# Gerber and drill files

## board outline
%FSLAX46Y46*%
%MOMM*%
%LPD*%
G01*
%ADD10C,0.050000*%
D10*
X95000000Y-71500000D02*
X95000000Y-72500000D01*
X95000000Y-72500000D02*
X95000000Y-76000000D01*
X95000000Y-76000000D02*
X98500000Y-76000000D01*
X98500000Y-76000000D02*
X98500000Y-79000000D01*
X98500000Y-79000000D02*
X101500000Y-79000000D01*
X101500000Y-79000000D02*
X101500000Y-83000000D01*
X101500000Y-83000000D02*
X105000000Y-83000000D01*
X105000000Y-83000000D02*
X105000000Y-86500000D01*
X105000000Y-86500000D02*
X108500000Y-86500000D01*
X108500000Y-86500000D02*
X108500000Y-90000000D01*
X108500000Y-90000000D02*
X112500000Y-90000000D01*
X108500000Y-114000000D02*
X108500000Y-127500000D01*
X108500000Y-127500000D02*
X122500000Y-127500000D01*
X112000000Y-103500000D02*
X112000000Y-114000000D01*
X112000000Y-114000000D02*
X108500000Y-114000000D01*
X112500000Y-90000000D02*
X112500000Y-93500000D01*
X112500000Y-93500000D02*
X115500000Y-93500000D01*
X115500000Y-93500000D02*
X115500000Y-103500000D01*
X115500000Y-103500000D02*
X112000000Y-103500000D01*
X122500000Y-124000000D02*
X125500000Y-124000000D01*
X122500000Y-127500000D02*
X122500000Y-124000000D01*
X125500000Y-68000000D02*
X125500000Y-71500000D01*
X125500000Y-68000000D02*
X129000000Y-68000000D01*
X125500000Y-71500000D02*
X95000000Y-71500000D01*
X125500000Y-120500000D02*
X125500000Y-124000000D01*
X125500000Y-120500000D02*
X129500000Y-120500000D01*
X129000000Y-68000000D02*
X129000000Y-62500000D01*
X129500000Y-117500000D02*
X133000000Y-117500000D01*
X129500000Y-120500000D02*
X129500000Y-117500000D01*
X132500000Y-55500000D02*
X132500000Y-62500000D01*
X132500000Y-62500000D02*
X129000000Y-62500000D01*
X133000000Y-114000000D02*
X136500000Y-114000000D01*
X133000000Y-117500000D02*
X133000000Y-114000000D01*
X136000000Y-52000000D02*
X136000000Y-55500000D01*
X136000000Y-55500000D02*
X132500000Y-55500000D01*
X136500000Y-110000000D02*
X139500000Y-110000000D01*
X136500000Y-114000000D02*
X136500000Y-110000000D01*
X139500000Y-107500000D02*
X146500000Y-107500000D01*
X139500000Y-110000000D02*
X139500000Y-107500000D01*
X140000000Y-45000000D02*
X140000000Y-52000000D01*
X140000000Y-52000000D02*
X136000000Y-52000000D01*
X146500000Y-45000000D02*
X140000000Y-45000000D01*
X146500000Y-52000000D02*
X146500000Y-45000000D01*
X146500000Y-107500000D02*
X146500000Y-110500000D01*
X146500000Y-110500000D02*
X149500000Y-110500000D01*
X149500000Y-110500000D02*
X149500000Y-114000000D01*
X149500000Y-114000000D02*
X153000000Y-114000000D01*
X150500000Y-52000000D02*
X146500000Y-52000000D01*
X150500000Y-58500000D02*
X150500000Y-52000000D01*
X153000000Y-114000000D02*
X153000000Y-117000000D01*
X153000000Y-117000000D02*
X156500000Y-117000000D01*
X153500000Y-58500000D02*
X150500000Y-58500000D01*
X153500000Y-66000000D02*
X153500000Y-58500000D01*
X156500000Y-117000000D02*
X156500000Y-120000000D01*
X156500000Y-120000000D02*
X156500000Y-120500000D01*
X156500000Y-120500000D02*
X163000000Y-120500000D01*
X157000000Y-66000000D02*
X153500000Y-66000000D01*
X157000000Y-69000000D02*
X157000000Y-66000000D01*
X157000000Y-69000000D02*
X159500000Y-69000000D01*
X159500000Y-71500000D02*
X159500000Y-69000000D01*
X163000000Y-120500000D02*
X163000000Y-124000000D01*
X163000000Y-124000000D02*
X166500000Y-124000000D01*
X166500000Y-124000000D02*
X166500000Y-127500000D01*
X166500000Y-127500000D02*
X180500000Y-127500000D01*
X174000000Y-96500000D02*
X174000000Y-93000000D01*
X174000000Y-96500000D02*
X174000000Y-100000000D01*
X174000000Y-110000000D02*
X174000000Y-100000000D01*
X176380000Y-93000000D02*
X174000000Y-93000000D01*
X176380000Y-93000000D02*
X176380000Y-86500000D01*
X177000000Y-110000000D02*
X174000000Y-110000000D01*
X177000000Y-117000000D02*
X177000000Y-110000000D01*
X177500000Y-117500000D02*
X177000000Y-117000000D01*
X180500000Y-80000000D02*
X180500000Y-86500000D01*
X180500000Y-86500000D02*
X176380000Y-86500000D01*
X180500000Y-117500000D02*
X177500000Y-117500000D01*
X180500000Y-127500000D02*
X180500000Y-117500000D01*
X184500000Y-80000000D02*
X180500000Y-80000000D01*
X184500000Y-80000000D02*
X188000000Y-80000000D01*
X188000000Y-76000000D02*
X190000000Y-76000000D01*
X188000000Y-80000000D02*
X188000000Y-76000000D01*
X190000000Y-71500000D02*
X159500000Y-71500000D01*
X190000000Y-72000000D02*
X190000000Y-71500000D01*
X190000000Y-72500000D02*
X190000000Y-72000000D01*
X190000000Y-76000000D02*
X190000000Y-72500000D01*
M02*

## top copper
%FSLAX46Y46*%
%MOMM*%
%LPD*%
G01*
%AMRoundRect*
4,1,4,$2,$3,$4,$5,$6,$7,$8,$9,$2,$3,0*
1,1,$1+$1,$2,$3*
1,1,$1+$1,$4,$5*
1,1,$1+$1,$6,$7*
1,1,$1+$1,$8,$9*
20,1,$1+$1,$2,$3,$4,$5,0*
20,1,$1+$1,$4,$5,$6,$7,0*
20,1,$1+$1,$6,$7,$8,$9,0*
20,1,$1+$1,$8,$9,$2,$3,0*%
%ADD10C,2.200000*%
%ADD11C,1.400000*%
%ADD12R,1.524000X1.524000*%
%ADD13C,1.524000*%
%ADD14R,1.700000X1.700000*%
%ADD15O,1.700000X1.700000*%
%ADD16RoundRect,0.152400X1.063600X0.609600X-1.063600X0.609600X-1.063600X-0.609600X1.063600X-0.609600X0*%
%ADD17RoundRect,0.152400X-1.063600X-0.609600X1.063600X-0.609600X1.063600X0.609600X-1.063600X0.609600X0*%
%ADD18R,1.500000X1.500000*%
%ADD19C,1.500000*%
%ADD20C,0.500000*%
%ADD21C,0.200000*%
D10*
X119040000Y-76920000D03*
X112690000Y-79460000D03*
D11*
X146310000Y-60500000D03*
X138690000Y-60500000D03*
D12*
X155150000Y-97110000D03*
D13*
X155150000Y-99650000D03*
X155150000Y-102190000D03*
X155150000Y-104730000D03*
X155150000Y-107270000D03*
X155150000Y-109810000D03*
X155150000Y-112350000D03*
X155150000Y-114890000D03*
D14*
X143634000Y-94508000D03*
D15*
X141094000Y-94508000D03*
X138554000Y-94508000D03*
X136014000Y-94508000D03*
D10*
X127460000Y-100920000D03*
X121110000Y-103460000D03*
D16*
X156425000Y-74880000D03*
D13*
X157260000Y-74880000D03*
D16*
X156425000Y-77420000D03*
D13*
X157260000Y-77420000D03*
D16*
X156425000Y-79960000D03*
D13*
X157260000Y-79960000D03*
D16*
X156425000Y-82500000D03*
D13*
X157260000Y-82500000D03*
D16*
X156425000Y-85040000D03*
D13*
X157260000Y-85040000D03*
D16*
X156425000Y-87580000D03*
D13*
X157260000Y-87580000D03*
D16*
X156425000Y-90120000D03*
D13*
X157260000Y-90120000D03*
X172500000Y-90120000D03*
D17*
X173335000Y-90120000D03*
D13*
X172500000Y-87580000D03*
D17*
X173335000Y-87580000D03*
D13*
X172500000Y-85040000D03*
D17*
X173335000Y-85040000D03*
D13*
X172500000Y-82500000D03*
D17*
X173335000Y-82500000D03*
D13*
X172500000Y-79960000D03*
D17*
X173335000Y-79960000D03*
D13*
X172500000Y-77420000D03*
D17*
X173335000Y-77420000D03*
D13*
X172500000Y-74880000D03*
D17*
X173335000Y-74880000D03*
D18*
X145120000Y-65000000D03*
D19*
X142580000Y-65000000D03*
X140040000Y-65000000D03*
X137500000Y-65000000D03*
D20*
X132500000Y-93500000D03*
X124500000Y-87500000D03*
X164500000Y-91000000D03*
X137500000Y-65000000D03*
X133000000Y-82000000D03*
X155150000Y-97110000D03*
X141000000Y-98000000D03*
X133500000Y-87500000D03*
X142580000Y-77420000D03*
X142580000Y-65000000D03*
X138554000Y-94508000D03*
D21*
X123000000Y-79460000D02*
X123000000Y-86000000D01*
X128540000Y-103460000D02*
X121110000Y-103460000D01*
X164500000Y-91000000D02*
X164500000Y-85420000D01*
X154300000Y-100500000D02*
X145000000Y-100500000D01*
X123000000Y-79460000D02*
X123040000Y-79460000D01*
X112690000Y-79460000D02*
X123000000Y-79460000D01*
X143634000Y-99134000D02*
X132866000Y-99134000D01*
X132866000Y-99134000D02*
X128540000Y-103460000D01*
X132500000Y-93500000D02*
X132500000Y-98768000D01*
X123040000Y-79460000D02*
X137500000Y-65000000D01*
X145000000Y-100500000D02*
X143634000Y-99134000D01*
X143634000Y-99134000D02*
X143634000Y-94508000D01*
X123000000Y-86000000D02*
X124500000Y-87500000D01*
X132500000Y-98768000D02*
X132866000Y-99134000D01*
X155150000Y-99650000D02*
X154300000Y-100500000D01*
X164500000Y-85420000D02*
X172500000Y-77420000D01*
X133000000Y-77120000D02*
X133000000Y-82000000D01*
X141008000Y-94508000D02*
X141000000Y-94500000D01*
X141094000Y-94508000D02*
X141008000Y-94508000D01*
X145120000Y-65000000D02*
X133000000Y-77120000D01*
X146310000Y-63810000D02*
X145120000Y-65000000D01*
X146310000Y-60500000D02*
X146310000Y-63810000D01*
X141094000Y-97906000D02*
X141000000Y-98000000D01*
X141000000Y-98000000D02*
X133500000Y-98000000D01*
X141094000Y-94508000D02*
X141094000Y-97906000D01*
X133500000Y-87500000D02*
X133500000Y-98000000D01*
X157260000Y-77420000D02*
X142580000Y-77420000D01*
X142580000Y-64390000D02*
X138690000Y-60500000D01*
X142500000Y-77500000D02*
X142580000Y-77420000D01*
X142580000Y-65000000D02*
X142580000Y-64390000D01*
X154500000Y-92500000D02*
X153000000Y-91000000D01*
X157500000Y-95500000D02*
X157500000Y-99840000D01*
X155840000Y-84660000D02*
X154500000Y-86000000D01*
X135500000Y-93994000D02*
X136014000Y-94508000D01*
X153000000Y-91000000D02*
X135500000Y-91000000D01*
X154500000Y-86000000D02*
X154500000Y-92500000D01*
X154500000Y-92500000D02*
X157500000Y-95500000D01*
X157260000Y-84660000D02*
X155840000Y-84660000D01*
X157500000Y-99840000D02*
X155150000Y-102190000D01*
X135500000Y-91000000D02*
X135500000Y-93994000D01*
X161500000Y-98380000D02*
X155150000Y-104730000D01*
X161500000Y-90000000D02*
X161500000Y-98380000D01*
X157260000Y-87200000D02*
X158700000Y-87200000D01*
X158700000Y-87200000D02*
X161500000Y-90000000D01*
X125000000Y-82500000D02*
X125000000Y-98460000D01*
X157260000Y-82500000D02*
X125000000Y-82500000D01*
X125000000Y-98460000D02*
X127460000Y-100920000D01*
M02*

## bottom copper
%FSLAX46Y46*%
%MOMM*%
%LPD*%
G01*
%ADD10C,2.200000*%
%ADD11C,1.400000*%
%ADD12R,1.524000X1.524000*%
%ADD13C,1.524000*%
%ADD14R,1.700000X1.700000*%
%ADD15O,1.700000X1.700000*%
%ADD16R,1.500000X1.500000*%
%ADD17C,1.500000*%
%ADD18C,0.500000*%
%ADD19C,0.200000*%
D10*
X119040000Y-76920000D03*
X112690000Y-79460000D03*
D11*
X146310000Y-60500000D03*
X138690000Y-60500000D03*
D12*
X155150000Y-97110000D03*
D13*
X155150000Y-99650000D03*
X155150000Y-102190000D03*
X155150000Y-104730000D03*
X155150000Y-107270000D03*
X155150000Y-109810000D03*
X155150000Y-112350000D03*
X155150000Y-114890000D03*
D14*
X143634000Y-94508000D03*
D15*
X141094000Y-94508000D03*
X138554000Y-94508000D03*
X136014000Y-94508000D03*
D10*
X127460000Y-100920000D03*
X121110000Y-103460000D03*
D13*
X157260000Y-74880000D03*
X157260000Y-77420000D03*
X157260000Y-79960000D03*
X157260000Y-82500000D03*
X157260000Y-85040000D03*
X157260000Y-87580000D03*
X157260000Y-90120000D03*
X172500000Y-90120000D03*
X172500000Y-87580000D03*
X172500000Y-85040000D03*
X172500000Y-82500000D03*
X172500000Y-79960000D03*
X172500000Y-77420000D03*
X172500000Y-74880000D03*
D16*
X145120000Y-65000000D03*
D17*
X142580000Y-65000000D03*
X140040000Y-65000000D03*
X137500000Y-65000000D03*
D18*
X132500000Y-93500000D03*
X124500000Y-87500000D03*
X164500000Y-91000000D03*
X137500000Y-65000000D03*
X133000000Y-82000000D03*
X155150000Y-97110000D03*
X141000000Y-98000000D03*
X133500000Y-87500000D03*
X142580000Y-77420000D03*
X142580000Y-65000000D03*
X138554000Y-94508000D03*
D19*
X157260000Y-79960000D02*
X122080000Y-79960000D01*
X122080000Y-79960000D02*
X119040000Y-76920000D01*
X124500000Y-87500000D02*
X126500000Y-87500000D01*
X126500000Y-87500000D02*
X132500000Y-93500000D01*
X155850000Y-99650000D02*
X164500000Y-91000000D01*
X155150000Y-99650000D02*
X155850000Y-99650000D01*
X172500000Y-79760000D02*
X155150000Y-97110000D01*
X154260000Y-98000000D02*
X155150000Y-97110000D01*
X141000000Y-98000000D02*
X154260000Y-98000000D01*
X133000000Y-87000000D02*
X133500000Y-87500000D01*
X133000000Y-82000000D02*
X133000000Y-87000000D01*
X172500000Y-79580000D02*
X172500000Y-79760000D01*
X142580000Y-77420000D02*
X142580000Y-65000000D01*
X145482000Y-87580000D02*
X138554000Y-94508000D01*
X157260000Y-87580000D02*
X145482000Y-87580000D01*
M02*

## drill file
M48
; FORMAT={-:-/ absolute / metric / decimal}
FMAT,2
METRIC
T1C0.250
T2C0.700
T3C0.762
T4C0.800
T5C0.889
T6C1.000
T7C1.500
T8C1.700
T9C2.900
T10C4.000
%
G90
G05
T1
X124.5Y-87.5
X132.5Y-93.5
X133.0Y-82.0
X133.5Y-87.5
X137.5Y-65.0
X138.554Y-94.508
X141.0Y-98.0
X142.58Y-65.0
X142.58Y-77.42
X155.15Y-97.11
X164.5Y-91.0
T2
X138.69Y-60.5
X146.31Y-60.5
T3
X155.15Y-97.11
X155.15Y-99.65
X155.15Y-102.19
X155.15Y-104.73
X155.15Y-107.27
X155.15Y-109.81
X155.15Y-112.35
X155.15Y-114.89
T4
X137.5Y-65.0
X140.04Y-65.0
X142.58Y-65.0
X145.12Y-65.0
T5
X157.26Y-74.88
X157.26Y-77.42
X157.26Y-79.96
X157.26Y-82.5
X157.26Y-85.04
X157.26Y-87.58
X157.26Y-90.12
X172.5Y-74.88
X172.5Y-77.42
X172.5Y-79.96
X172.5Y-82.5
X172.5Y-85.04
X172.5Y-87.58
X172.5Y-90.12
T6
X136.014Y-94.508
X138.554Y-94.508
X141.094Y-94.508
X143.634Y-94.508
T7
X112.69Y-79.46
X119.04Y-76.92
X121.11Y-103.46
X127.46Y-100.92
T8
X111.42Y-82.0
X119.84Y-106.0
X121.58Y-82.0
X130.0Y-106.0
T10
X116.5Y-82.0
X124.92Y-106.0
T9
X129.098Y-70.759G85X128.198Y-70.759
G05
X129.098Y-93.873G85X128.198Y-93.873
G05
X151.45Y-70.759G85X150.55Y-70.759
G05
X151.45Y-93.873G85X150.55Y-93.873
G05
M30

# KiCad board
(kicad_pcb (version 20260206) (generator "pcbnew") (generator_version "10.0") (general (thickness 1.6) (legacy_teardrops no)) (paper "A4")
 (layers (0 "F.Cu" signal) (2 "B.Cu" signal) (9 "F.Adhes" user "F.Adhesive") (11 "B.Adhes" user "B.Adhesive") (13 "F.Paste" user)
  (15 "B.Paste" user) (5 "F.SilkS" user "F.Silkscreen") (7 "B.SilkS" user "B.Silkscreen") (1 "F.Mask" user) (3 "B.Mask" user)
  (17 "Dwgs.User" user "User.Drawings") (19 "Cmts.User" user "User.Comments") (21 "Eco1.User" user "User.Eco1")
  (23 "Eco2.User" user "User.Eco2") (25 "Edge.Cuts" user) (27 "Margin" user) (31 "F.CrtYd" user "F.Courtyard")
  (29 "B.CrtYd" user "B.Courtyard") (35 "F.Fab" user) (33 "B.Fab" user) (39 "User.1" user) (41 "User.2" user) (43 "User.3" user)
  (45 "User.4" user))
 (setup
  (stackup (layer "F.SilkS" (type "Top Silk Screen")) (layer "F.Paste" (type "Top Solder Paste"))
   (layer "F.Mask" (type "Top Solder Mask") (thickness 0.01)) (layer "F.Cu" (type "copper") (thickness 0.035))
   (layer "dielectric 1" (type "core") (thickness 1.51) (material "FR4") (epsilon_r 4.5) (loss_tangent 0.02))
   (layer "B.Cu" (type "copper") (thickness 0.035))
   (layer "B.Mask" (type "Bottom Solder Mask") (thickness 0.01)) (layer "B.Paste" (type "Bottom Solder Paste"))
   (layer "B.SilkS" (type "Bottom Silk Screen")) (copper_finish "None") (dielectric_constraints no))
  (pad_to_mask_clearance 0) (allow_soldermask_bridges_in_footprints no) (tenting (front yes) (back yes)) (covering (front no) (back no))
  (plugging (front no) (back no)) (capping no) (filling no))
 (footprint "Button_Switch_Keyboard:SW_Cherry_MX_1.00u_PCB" (layer "F.Cu") (at 119.04 76.92)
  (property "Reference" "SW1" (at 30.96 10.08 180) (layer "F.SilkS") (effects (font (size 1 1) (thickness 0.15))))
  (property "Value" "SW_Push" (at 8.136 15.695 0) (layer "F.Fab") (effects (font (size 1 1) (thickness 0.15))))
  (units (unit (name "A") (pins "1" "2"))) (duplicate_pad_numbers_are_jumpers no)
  (pad "" np_thru_hole circle (at -7.62 5.08) (size 1.7 1.7) (drill 1.7) (layers "*.Cu" "*.Mask"))
  (pad "" np_thru_hole circle (at -2.54 5.08) (size 4 4) (drill 4) (layers "*.Cu" "*.Mask"))
  (pad "" np_thru_hole circle (at 2.54 5.08) (size 1.7 1.7) (drill 1.7) (layers "*.Cu" "*.Mask"))
  (pad "1" thru_hole circle (at 0 0) (size 2.2 2.2) (drill 1.5) (layers "*.Cu" "*.Mask") (remove_unused_layers no) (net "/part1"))
  (pad "2" thru_hole circle (at -6.35 2.54) (size 2.2 2.2) (drill 1.5) (layers "*.Cu" "*.Mask") (remove_unused_layers no) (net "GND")))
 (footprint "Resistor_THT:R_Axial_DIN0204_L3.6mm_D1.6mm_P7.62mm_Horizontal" (layer "F.Cu") (at 146.31 60.5 180)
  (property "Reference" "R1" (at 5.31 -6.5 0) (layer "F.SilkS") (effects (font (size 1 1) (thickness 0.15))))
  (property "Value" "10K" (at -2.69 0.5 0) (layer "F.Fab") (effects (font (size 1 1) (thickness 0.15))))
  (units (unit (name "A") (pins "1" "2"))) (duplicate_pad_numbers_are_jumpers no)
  (pad "1" thru_hole circle (at 0 0 180) (size 1.4 1.4) (drill 0.7) (layers "*.Cu" "*.Mask") (remove_unused_layers no) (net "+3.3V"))
  (pad "2" thru_hole circle (at 7.62 0 180) (size 1.4 1.4) (drill 0.7) (layers "*.Cu" "*.Mask") (remove_unused_layers no)
   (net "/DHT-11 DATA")))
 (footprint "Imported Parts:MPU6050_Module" (layer "F.Cu") (at 155.15 97.11)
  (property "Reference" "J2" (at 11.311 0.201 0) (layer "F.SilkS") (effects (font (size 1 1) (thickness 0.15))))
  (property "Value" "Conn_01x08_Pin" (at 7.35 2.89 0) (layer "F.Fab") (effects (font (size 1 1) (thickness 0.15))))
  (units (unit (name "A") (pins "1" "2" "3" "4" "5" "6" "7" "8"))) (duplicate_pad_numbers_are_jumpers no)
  (pad "1" thru_hole rect (at 0 0) (size 1.524 1.524) (drill 0.762) (layers "*.Cu" "*.Mask") (remove_unused_layers no) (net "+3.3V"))
  (pad "2" thru_hole circle (at 0 2.54) (size 1.524 1.524) (drill 0.762) (layers "*.Cu" "*.Mask") (remove_unused_layers no) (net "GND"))
  (pad "3" thru_hole circle (at 0 5.08) (size 1.524 1.524) (drill 0.762) (layers "*.Cu" "*.Mask") (remove_unused_layers no) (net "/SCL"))
  (pad "4" thru_hole circle (at 0 7.62) (size 1.524 1.524) (drill 0.762) (layers "*.Cu" "*.Mask") (remove_unused_layers no) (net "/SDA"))
  (pad "5" thru_hole circle (at 0 10.16) (size 1.524 1.524) (drill 0.762) (layers "*.Cu" "*.Mask") (remove_unused_layers no)
   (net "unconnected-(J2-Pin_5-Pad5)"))
  (pad "6" thru_hole circle (at 0 12.7) (size 1.524 1.524) (drill 0.762) (layers "*.Cu" "*.Mask") (remove_unused_layers no)
   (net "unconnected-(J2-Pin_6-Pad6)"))
  (pad "7" thru_hole circle (at 0 15.24) (size 1.524 1.524) (drill 0.762) (layers "*.Cu" "*.Mask") (remove_unused_layers no)
   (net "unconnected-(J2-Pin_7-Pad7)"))
  (pad "8" thru_hole circle (at 0 17.78) (size 1.524 1.524) (drill 0.762) (layers "*.Cu" "*.Mask") (remove_unused_layers no)
   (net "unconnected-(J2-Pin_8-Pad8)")))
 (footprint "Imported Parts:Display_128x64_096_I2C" (layer "F.Cu") (at 139.824 94.508 180)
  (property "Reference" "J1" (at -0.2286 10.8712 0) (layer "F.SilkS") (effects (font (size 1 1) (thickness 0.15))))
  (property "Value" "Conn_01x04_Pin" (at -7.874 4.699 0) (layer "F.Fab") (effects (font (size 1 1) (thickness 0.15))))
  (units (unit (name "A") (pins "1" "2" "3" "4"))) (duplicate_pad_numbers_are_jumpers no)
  (pad "" np_thru_hole oval (at -11.176 0.635 180) (size 3.8 2.9) (drill oval 3.8 2.9) (layers "*.Cu" "*.Mask"))
  (pad "" np_thru_hole oval (at -11.176 23.749 180) (size 3.8 2.9) (drill oval 3.8 2.9) (layers "*.Cu" "*.Mask"))
  (pad "" np_thru_hole oval (at 11.176 0.635 180) (size 3.8 2.9) (drill oval 3.8 2.9) (layers "*.Cu" "*.Mask"))
  (pad "" np_thru_hole oval (at 11.176 23.749 180) (size 3.8 2.9) (drill oval 3.8 2.9) (layers "*.Cu" "*.Mask"))
  (pad "1" thru_hole rect (at -3.81 0 270) (size 1.7 1.7) (drill 1) (layers "*.Cu" "*.Mask") (remove_unused_layers no) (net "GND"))
  (pad "2" thru_hole oval (at -1.27 0 270) (size 1.7 1.7) (drill 1) (layers "*.Cu" "*.Mask") (remove_unused_layers no) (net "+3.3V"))
  (pad "3" thru_hole oval (at 1.27 0 270) (size 1.7 1.7) (drill 1) (layers "*.Cu" "*.Mask") (remove_unused_layers no) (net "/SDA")
   (solder_mask_margin 0))
  (pad "4" thru_hole oval (at 3.81 0 270) (size 1.7 1.7) (drill 1) (layers "*.Cu" "*.Mask") (remove_unused_layers no) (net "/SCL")))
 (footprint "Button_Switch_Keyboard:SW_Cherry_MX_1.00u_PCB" (layer "F.Cu") (at 127.46 100.92)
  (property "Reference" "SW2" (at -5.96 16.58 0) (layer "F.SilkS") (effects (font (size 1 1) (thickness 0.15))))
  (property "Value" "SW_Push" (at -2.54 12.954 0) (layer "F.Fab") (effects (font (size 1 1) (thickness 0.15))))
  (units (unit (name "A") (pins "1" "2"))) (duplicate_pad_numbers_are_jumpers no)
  (pad "" np_thru_hole circle (at -7.62 5.08) (size 1.7 1.7) (drill 1.7) (layers "*.Cu" "*.Mask"))
  (pad "" np_thru_hole circle (at -2.54 5.08) (size 4 4) (drill 4) (layers "*.Cu" "*.Mask"))
  (pad "" np_thru_hole circle (at 2.54 5.08) (size 1.7 1.7) (drill 1.7) (layers "*.Cu" "*.Mask"))
  (pad "1" thru_hole circle (at 0 0) (size 2.2 2.2) (drill 1.5) (layers "*.Cu" "*.Mask") (remove_unused_layers no) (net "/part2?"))
  (pad "2" thru_hole circle (at -6.35 2.54) (size 2.2 2.2) (drill 1.5) (layers "*.Cu" "*.Mask") (remove_unused_layers no) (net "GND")))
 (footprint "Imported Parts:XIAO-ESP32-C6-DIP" (layer "F.Cu") (at 164.88 82.5 90)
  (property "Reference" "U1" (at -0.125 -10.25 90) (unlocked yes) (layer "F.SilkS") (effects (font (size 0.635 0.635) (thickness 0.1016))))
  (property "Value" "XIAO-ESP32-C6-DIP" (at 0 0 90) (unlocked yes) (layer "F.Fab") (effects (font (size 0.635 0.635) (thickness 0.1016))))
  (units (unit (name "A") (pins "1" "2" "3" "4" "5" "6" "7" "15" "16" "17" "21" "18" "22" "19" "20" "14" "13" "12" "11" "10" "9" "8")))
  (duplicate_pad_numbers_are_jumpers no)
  (pad "1" smd roundrect (at 7.62 -8.455 180) (size 2.432 1.524) (layers "F.Cu" "F.Mask") (roundrect_rratio 0.1)
   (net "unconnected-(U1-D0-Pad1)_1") (thermal_bridge_angle 45))
  (pad "1" thru_hole circle (at 7.62 -7.62 180) (size 1.524 1.524) (drill 0.889) (layers "*.Cu" "*.Mask") (remove_unused_layers no)
   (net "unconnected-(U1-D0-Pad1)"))
  (pad "2" smd roundrect (at 5.08 -8.455 180) (size 2.432 1.524) (layers "F.Cu" "F.Mask") (roundrect_rratio 0.1) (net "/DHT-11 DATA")
   (thermal_bridge_angle 45))
  (pad "2" thru_hole circle (at 5.08 -7.62 180) (size 1.524 1.524) (drill 0.889) (layers "*.Cu" "*.Mask") (remove_unused_layers no)
   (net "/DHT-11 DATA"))
  (pad "3" smd roundrect (at 2.54 -8.455 180) (size 2.432 1.524) (layers "F.Cu" "F.Mask") (roundrect_rratio 0.1) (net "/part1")
   (thermal_bridge_angle 45))
  (pad "3" thru_hole circle (at 2.54 -7.62 180) (size 1.524 1.524) (drill 0.889) (layers "*.Cu" "*.Mask") (remove_unused_layers no)
   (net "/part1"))
  (pad "4" smd roundrect (at 0 -8.455 180) (size 2.432 1.524) (layers "F.Cu" "F.Mask") (roundrect_rratio 0.1) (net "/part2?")
   (thermal_bridge_angle 45))
  (pad "4" thru_hole circle (at 0 -7.62 180) (size 1.524 1.524) (drill 0.889) (layers "*.Cu" "*.Mask") (remove_unused_layers no)
   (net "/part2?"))
  (pad "5" smd roundrect (at -2.54 -8.455 180) (size 2.432 1.524) (layers "F.Cu" "F.Mask") (roundrect_rratio 0.1) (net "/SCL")
   (thermal_bridge_angle 45))
  (pad "5" thru_hole circle (at -2.54 -7.62 180) (size 1.524 1.524) (drill 0.889) (layers "*.Cu" "*.Mask") (remove_unused_layers no)
   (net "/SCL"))
  (pad "6" smd roundrect (at -5.08 -8.455 180) (size 2.432 1.524) (layers "F.Cu" "F.Mask") (roundrect_rratio 0.1) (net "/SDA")
   (thermal_bridge_angle 45))
  (pad "6" thru_hole circle (at -5.08 -7.62 180) (size 1.524 1.524) (drill 0.889) (layers "*.Cu" "*.Mask") (remove_unused_layers no)
   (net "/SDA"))
  (pad "7" smd roundrect (at -7.62 -8.455 180) (size 2.432 1.524) (layers "F.Cu" "F.Mask") (roundrect_rratio 0.1)
   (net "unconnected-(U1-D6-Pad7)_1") (thermal_bridge_angle 45))
  (pad "7" thru_hole circle (at -7.62 -7.62 180) (size 1.524 1.524) (drill 0.889) (layers "*.Cu" "*.Mask") (remove_unused_layers no)
   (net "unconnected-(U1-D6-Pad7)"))
  (pad "8" thru_hole circle (at -7.62 7.62) (size 1.524 1.524) (drill 0.889) (layers "*.Cu" "*.Mask") (remove_unused_layers no)
   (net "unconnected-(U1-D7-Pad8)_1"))
  (pad "8" smd roundrect (at -7.62 8.455) (size 2.432 1.524) (layers "F.Cu" "F.Mask") (roundrect_rratio 0.1)
   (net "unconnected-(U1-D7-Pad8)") (thermal_bridge_angle 45))
  (pad "9" thru_hole circle (at -5.08 7.62) (size 1.524 1.524) (drill 0.889) (layers "*.Cu" "*.Mask") (remove_unused_layers no)
   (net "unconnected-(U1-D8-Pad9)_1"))
  (pad "9" smd roundrect (at -5.08 8.455) (size 2.432 1.524) (layers "F.Cu" "F.Mask") (roundrect_rratio 0.1)
   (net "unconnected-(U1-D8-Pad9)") (thermal_bridge_angle 45))
  (pad "10" thru_hole circle (at -2.54 7.62) (size 1.524 1.524) (drill 0.889) (layers "*.Cu" "*.Mask") (remove_unused_layers no)
   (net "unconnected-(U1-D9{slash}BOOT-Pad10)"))
  (pad "10" smd roundrect (at -2.54 8.455) (size 2.432 1.524) (layers "F.Cu" "F.Mask") (roundrect_rratio 0.1)
   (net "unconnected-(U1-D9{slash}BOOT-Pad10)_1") (thermal_bridge_angle 45))
  (pad "11" thru_hole circle (at 0 7.62) (size 1.524 1.524) (drill 0.889) (layers "*.Cu" "*.Mask") (remove_unused_layers no)
   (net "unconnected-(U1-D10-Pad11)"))
  (pad "11" smd roundrect (at 0 8.455) (size 2.432 1.524) (layers "F.Cu" "F.Mask") (roundrect_rratio 0.1)
   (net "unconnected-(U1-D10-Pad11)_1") (thermal_bridge_angle 45))
  (pad "12" thru_hole circle (at 2.54 7.62) (size 1.524 1.524) (drill 0.889) (layers "*.Cu" "*.Mask") (remove_unused_layers no)
   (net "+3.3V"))
  (pad "12" smd roundrect (at 2.54 8.455) (size 2.432 1.524) (layers "F.Cu" "F.Mask") (roundrect_rratio 0.1) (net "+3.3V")
   (thermal_bridge_angle 45))
  (pad "13" thru_hole circle (at 5.08 7.62) (size 1.524 1.524) (drill 0.889) (layers "*.Cu" "*.Mask") (remove_unused_layers no) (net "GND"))
  (pad "13" smd roundrect (at 5.08 8.455) (size 2.432 1.524) (layers "F.Cu" "F.Mask") (roundrect_rratio 0.1) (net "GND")
   (thermal_bridge_angle 45))
  (pad "14" thru_hole circle (at 7.62 7.62) (size 1.524 1.524) (drill 0.889) (layers "*.Cu" "*.Mask") (remove_unused_layers no) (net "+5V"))
  (pad "14" smd roundrect (at 7.62 8.455) (size 2.432 1.524) (layers "F.Cu" "F.Mask") (roundrect_rratio 0.1) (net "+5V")
   (thermal_bridge_angle 45)))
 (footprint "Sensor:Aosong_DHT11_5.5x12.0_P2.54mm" (layer "F.Cu") (at 145.12 65 -90)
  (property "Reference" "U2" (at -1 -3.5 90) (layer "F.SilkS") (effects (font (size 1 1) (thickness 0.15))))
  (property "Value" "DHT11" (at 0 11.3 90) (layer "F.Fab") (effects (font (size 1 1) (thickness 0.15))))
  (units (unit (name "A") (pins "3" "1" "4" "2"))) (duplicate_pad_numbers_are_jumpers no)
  (pad "1" thru_hole rect (at 0 0 270) (size 1.5 1.5) (drill 0.8) (layers "*.Cu" "*.Mask") (remove_unused_layers no) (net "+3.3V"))
  (pad "2" thru_hole circle (at 0 2.54 270) (size 1.5 1.5) (drill 0.8) (layers "*.Cu" "*.Mask") (remove_unused_layers no)
   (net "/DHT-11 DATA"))
  (pad "3" thru_hole circle (at 0 5.08 270) (size 1.5 1.5) (drill 0.8) (layers "*.Cu" "*.Mask") (remove_unused_layers no)
   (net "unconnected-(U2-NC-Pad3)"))
  (pad "4" thru_hole circle (at 0 7.62 270) (size 1.5 1.5) (drill 0.8) (layers "*.Cu" "*.Mask") (remove_unused_layers no) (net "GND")))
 (gr_line (start 95 71.5) (end 95 72.5) (stroke (width 0.05) (type default)) (layer "Edge.Cuts"))
 (gr_line (start 95 72.5) (end 95 76) (stroke (width 0.05) (type default)) (layer "Edge.Cuts"))
 (gr_line (start 95 76) (end 98.5 76) (stroke (width 0.05) (type default)) (layer "Edge.Cuts"))
 (gr_line (start 98.5 76) (end 98.5 79) (stroke (width 0.05) (type default)) (layer "Edge.Cuts"))
 (gr_line (start 98.5 79) (end 101.5 79) (stroke (width 0.05) (type default)) (layer "Edge.Cuts"))
 (gr_line (start 101.5 79) (end 101.5 83) (stroke (width 0.05) (type default)) (layer "Edge.Cuts"))
 (gr_line (start 101.5 83) (end 105 83) (stroke (width 0.05) (type default)) (layer "Edge.Cuts"))
 (gr_line (start 105 83) (end 105 86.5) (stroke (width 0.05) (type default)) (layer "Edge.Cuts"))
 (gr_line (start 105 86.5) (end 108.5 86.5) (stroke (width 0.05) (type default)) (layer "Edge.Cuts"))
 (gr_line (start 108.5 86.5) (end 108.5 90) (stroke (width 0.05) (type default)) (layer "Edge.Cuts"))
 (gr_line (start 108.5 90) (end 112.5 90) (stroke (width 0.05) (type default)) (layer "Edge.Cuts"))
 (gr_line (start 108.5 114) (end 108.5 127.5) (stroke (width 0.05) (type default)) (layer "Edge.Cuts"))
 (gr_line (start 108.5 127.5) (end 122.5 127.5) (stroke (width 0.05) (type default)) (layer "Edge.Cuts"))
 (gr_line (start 112 103.5) (end 112 114) (stroke (width 0.05) (type default)) (layer "Edge.Cuts"))
 (gr_line (start 112 114) (end 108.5 114) (stroke (width 0.05) (type default)) (layer "Edge.Cuts"))
 (gr_line (start 112.5 90) (end 112.5 93.5) (stroke (width 0.05) (type default)) (layer "Edge.Cuts"))
 (gr_line (start 112.5 93.5) (end 115.5 93.5) (stroke (width 0.05) (type default)) (layer "Edge.Cuts"))
 (gr_line (start 115.5 93.5) (end 115.5 103.5) (stroke (width 0.05) (type default)) (layer "Edge.Cuts"))
 (gr_line (start 115.5 103.5) (end 112 103.5) (stroke (width 0.05) (type default)) (layer "Edge.Cuts"))
 (gr_line (start 122.5 124) (end 125.5 124) (stroke (width 0.05) (type default)) (layer "Edge.Cuts"))
 (gr_line (start 122.5 127.5) (end 122.5 124) (stroke (width 0.05) (type default)) (layer "Edge.Cuts"))
 (gr_line (start 125.5 68) (end 125.5 71.5) (stroke (width 0.05) (type default)) (layer "Edge.Cuts"))
 (gr_line (start 125.5 68) (end 129 68) (stroke (width 0.05) (type default)) (layer "Edge.Cuts"))
 (gr_line (start 125.5 71.5) (end 95 71.5) (stroke (width 0.05) (type default)) (layer "Edge.Cuts"))
 (gr_line (start 125.5 120.5) (end 125.5 124) (stroke (width 0.05) (type default)) (layer "Edge.Cuts"))
 (gr_line (start 125.5 120.5) (end 129.5 120.5) (stroke (width 0.05) (type default)) (layer "Edge.Cuts"))
 (gr_line (start 129 68) (end 129 62.5) (stroke (width 0.05) (type default)) (layer "Edge.Cuts"))
 (gr_line (start 129.5 117.5) (end 133 117.5) (stroke (width 0.05) (type default)) (layer "Edge.Cuts"))
 (gr_line (start 129.5 120.5) (end 129.5 117.5) (stroke (width 0.05) (type default)) (layer "Edge.Cuts"))
 (gr_line (start 132.5 55.5) (end 132.5 62.5) (stroke (width 0.05) (type default)) (layer "Edge.Cuts"))
 (gr_line (start 132.5 62.5) (end 129 62.5) (stroke (width 0.05) (type default)) (layer "Edge.Cuts"))
 (gr_line (start 133 114) (end 136.5 114) (stroke (width 0.05) (type default)) (layer "Edge.Cuts"))
 (gr_line (start 133 117.5) (end 133 114) (stroke (width 0.05) (type default)) (layer "Edge.Cuts"))
 (gr_line (start 136 52) (end 136 55.5) (stroke (width 0.05) (type default)) (layer "Edge.Cuts"))
 (gr_line (start 136 55.5) (end 132.5 55.5) (stroke (width 0.05) (type default)) (layer "Edge.Cuts"))
 (gr_line (start 136.5 110) (end 139.5 110) (stroke (width 0.05) (type default)) (layer "Edge.Cuts"))
 (gr_line (start 136.5 114) (end 136.5 110) (stroke (width 0.05) (type default)) (layer "Edge.Cuts"))
 (gr_line (start 139.5 107.5) (end 146.5 107.5) (stroke (width 0.05) (type default)) (layer "Edge.Cuts"))
 (gr_line (start 139.5 110) (end 139.5 107.5) (stroke (width 0.05) (type default)) (layer "Edge.Cuts"))
 (gr_line (start 140 45) (end 140 52) (stroke (width 0.05) (type default)) (layer "Edge.Cuts"))
 (gr_line (start 140 52) (end 136 52) (stroke (width 0.05) (type default)) (layer "Edge.Cuts"))
 (gr_line (start 146.5 45) (end 140 45) (stroke (width 0.05) (type default)) (layer "Edge.Cuts"))
 (gr_line (start 146.5 52) (end 146.5 45) (stroke (width 0.05) (type default)) (layer "Edge.Cuts"))
 (gr_line (start 146.5 107.5) (end 146.5 110.5) (stroke (width 0.05) (type default)) (layer "Edge.Cuts"))
 (gr_line (start 146.5 110.5) (end 149.5 110.5) (stroke (width 0.05) (type default)) (layer "Edge.Cuts"))
 (gr_line (start 149.5 110.5) (end 149.5 114) (stroke (width 0.05) (type default)) (layer "Edge.Cuts"))
 (gr_line (start 149.5 114) (end 153 114) (stroke (width 0.05) (type default)) (layer "Edge.Cuts"))
 (gr_line (start 150.5 52) (end 146.5 52) (stroke (width 0.05) (type default)) (layer "Edge.Cuts"))
 (gr_line (start 150.5 58.5) (end 150.5 52) (stroke (width 0.05) (type default)) (layer "Edge.Cuts"))
 (gr_line (start 153 114) (end 153 117) (stroke (width 0.05) (type default)) (layer "Edge.Cuts"))
 (gr_line (start 153 117) (end 156.5 117) (stroke (width 0.05) (type default)) (layer "Edge.Cuts"))
 (gr_line (start 153.5 58.5) (end 150.5 58.5) (stroke (width 0.05) (type default)) (layer "Edge.Cuts"))
 (gr_line (start 153.5 66) (end 153.5 58.5) (stroke (width 0.05) (type default)) (layer "Edge.Cuts"))
 (gr_line (start 156.5 117) (end 156.5 120) (stroke (width 0.05) (type default)) (layer "Edge.Cuts"))
 (gr_line (start 156.5 120) (end 156.5 120.5) (stroke (width 0.05) (type default)) (layer "Edge.Cuts"))
 (gr_line (start 156.5 120.5) (end 163 120.5) (stroke (width 0.05) (type default)) (layer "Edge.Cuts"))
 (gr_line (start 157 66) (end 153.5 66) (stroke (width 0.05) (type default)) (layer "Edge.Cuts"))
 (gr_line (start 157 69) (end 157 66) (stroke (width 0.05) (type default)) (layer "Edge.Cuts"))
 (gr_line (start 157 69) (end 159.5 69) (stroke (width 0.05) (type default)) (layer "Edge.Cuts"))
 (gr_line (start 159.5 71.5) (end 159.5 69) (stroke (width 0.05) (type default)) (layer "Edge.Cuts"))
 (gr_line (start 163 120.5) (end 163 124) (stroke (width 0.05) (type default)) (layer "Edge.Cuts"))
 (gr_line (start 163 124) (end 166.5 124) (stroke (width 0.05) (type default)) (layer "Edge.Cuts"))
 (gr_line (start 166.5 124) (end 166.5 127.5) (stroke (width 0.05) (type default)) (layer "Edge.Cuts"))
 (gr_line (start 166.5 127.5) (end 180.5 127.5) (stroke (width 0.05) (type default)) (layer "Edge.Cuts"))
 (gr_line (start 174 96.5) (end 174 93) (stroke (width 0.05) (type default)) (layer "Edge.Cuts"))
 (gr_line (start 174 96.5) (end 174 100) (stroke (width 0.05) (type default)) (layer "Edge.Cuts"))
 (gr_line (start 174 110) (end 174 100) (stroke (width 0.05) (type default)) (layer "Edge.Cuts"))
 (gr_line (start 176.38 93) (end 174 93) (stroke (width 0.05) (type default)) (layer "Edge.Cuts"))
 (gr_line (start 176.38 93) (end 176.38 86.5) (stroke (width 0.05) (type default)) (layer "Edge.Cuts"))
 (gr_line (start 177 110) (end 174 110) (stroke (width 0.05) (type default)) (layer "Edge.Cuts"))
 (gr_line (start 177 117) (end 177 110) (stroke (width 0.05) (type default)) (layer "Edge.Cuts"))
 (gr_line (start 177.5 117.5) (end 177 117) (stroke (width 0.05) (type default)) (layer "Edge.Cuts"))
 (gr_line (start 180.5 80) (end 180.5 86.5) (stroke (width 0.05) (type default)) (layer "Edge.Cuts"))
 (gr_line (start 180.5 86.5) (end 176.38 86.5) (stroke (width 0.05) (type default)) (layer "Edge.Cuts"))
 (gr_line (start 180.5 117.5) (end 177.5 117.5) (stroke (width 0.05) (type default)) (layer "Edge.Cuts"))
 (gr_line (start 180.5 127.5) (end 180.5 117.5) (stroke (width 0.05) (type default)) (layer "Edge.Cuts"))
 (gr_line (start 184.5 80) (end 180.5 80) (stroke (width 0.05) (type default)) (layer "Edge.Cuts"))
 (gr_line (start 184.5 80) (end 188 80) (stroke (width 0.05) (type default)) (layer "Edge.Cuts"))
 (gr_line (start 188 76) (end 190 76) (stroke (width 0.05) (type default)) (layer "Edge.Cuts"))
 (gr_line (start 188 80) (end 188 76) (stroke (width 0.05) (type default)) (layer "Edge.Cuts"))
 (gr_line (start 190 71.5) (end 159.5 71.5) (stroke (width 0.05) (type default)) (layer "Edge.Cuts"))
 (gr_line (start 190 72) (end 190 71.5) (stroke (width 0.05) (type default)) (layer "Edge.Cuts"))
 (gr_line (start 190 72.5) (end 190 72) (stroke (width 0.05) (type default)) (layer "Edge.Cuts"))
 (gr_line (start 190 76) (end 190 72.5) (stroke (width 0.05) (type default)) (layer "Edge.Cuts"))
 (segment (start 157.26 79.96) (end 122.08 79.96) (width 0.2) (layer "B.Cu") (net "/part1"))
 (segment (start 122.08 79.96) (end 119.04 76.92) (width 0.2) (layer "B.Cu") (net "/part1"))
 (segment (start 123 79.46) (end 123 86) (width 0.2) (layer "F.Cu") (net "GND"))
 (segment (start 128.54 103.46) (end 121.11 103.46) (width 0.2) (layer "F.Cu") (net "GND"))
 (segment (start 164.5 91) (end 164.5 85.42) (width 0.2) (layer "F.Cu") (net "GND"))
 (segment (start 154.3 100.5) (end 145 100.5) (width 0.2) (layer "F.Cu") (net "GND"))
 (segment (start 123 79.46) (end 123.04 79.46) (width 0.2) (layer "F.Cu") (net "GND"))
 (segment (start 112.69 79.46) (end 123 79.46) (width 0.2) (layer "F.Cu") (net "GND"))
 (segment (start 143.634 99.134) (end 132.866 99.134) (width 0.2) (layer "F.Cu") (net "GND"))
 (segment (start 132.866 99.134) (end 128.54 103.46) (width 0.2) (layer "F.Cu") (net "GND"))
 (segment (start 132.5 93.5) (end 132.5 98.768) (width 0.2) (layer "F.Cu") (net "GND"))
 (segment (start 123.04 79.46) (end 137.5 65) (width 0.2) (layer "F.Cu") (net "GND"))
 (segment (start 145 100.5) (end 143.634 99.134) (width 0.2) (layer "F.Cu") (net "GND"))
 (segment (start 143.634 99.134) (end 143.634 94.508) (width 0.2) (layer "F.Cu") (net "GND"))
 (segment (start 123 86) (end 124.5 87.5) (width 0.2) (layer "F.Cu") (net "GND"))
 (segment (start 132.5 98.768) (end 132.866 99.134) (width 0.2) (layer "F.Cu") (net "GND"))
 (segment (start 155.15 99.65) (end 154.3 100.5) (width 0.2) (layer "F.Cu") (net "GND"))
 (segment (start 164.5 85.42) (end 172.5 77.42) (width 0.2) (layer "F.Cu") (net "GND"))
 (via (at 132.5 93.5) (size 0.5) (drill 0.25) (layers "F.Cu" "B.Cu") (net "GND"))
 (via (at 124.5 87.5) (size 0.5) (drill 0.25) (layers "F.Cu" "B.Cu") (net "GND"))
 (via (at 164.5 91) (size 0.5) (drill 0.25) (layers "F.Cu" "B.Cu") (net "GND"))
 (via (at 137.5 65) (size 0.5) (drill 0.25) (layers "F.Cu" "B.Cu") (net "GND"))
 (segment (start 124.5 87.5) (end 126.5 87.5) (width 0.2) (layer "B.Cu") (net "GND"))
 (segment (start 126.5 87.5) (end 132.5 93.5) (width 0.2) (layer "B.Cu") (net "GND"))
 (segment (start 155.85 99.65) (end 164.5 91) (width 0.2) (layer "B.Cu") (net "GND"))
 (segment (start 155.15 99.65) (end 155.85 99.65) (width 0.2) (layer "B.Cu") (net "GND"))
 (segment (start 133 77.12) (end 133 82) (width 0.2) (layer "F.Cu") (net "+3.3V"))
 (segment (start 141.008 94.508) (end 141 94.5) (width 0.2) (layer "F.Cu") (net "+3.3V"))
 (segment (start 141.094 94.508) (end 141.008 94.508) (width 0.2) (layer "F.Cu") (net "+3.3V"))
 (segment (start 145.12 65) (end 133 77.12) (width 0.2) (layer "F.Cu") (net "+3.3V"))
 (segment (start 146.31 63.81) (end 145.12 65) (width 0.2) (layer "F.Cu") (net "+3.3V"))
 (segment (start 146.31 60.5) (end 146.31 63.81) (width 0.2) (layer "F.Cu") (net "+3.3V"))
 (segment (start 141.094 97.906) (end 141 98) (width 0.2) (layer "F.Cu") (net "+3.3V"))
 (segment (start 141 98) (end 133.5 98) (width 0.2) (layer "F.Cu") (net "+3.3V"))
 (segment (start 141.094 94.508) (end 141.094 97.906) (width 0.2) (layer "F.Cu") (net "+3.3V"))
 (segment (start 133.5 87.5) (end 133.5 98) (width 0.2) (layer "F.Cu") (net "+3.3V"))
 (via (at 133 82) (size 0.5) (drill 0.25) (layers "F.Cu" "B.Cu") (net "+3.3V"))
 (via (at 155.15 97.11) (size 0.5) (drill 0.25) (layers "F.Cu" "B.Cu") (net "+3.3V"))
 (via (at 141 98) (size 0.5) (drill 0.25) (layers "F.Cu" "B.Cu") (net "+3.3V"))
 (via (at 133.5 87.5) (size 0.5) (drill 0.25) (layers "F.Cu" "B.Cu") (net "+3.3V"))
 (segment (start 172.5 79.76) (end 155.15 97.11) (width 0.2) (layer "B.Cu") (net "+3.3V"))
 (segment (start 154.26 98) (end 155.15 97.11) (width 0.2) (layer "B.Cu") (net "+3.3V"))
 (segment (start 141 98) (end 154.26 98) (width 0.2) (layer "B.Cu") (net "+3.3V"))
 (segment (start 133 87) (end 133.5 87.5) (width 0.2) (layer "B.Cu") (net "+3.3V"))
 (segment (start 133 82) (end 133 87) (width 0.2) (layer "B.Cu") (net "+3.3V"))
 (segment (start 172.5 79.58) (end 172.5 79.76) (width 0.2) (layer "B.Cu") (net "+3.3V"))
 (segment (start 157.26 77.42) (end 142.58 77.42) (width 0.2) (layer "F.Cu") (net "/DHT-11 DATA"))
 (segment (start 142.58 64.39) (end 138.69 60.5) (width 0.2) (layer "F.Cu") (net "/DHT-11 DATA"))
 (segment (start 142.5 77.5) (end 142.58 77.42) (width 0.2) (layer "F.Cu") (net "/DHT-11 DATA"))
 (segment (start 142.58 65) (end 142.58 64.39) (width 0.2) (layer "F.Cu") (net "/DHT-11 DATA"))
 (via (at 142.58 77.42) (size 0.5) (drill 0.25) (layers "F.Cu" "B.Cu") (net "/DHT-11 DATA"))
 (via (at 142.58 65) (size 0.5) (drill 0.25) (layers "F.Cu" "B.Cu") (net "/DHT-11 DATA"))
 (segment (start 142.58 77.42) (end 142.58 65) (width 0.2) (layer "B.Cu") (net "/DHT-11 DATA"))
 (segment (start 154.5 92.5) (end 153 91) (width 0.2) (layer "F.Cu") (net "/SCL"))
 (segment (start 157.5 95.5) (end 157.5 99.84) (width 0.2) (layer "F.Cu") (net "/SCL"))
 (segment (start 155.84 84.66) (end 154.5 86) (width 0.2) (layer "F.Cu") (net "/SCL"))
 (segment (start 135.5 93.994) (end 136.014 94.508) (width 0.2) (layer "F.Cu") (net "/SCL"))
 (segment (start 153 91) (end 135.5 91) (width 0.2) (layer "F.Cu") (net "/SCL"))
 (segment (start 154.5 86) (end 154.5 92.5) (width 0.2) (layer "F.Cu") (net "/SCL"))
 (segment (start 154.5 92.5) (end 157.5 95.5) (width 0.2) (layer "F.Cu") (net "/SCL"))
 (segment (start 157.26 84.66) (end 155.84 84.66) (width 0.2) (layer "F.Cu") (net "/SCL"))
 (segment (start 157.5 99.84) (end 155.15 102.19) (width 0.2) (layer "F.Cu") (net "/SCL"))
 (segment (start 135.5 91) (end 135.5 93.994) (width 0.2) (layer "F.Cu") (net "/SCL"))
 (segment (start 161.5 98.38) (end 155.15 104.73) (width 0.2) (layer "F.Cu") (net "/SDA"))
 (segment (start 161.5 90) (end 161.5 98.38) (width 0.2) (layer "F.Cu") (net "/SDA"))
 (segment (start 157.26 87.2) (end 158.7 87.2) (width 0.2) (layer "F.Cu") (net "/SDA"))
 (segment (start 158.7 87.2) (end 161.5 90) (width 0.2) (layer "F.Cu") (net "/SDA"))
 (via (at 138.554 94.508) (size 0.5) (drill 0.25) (layers "F.Cu" "B.Cu") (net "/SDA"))
 (segment (start 145.482 87.58) (end 138.554 94.508) (width 0.2) (layer "B.Cu") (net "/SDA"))
 (segment (start 157.26 87.58) (end 145.482 87.58) (width 0.2) (layer "B.Cu") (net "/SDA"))
 (segment (start 125 82.5) (end 125 98.46) (width 0.2) (layer "F.Cu") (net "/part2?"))
 (segment (start 157.26 82.5) (end 125 82.5) (width 0.2) (layer "F.Cu") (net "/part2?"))
 (segment (start 125 98.46) (end 127.46 100.92) (width 0.2) (layer "F.Cu") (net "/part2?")))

